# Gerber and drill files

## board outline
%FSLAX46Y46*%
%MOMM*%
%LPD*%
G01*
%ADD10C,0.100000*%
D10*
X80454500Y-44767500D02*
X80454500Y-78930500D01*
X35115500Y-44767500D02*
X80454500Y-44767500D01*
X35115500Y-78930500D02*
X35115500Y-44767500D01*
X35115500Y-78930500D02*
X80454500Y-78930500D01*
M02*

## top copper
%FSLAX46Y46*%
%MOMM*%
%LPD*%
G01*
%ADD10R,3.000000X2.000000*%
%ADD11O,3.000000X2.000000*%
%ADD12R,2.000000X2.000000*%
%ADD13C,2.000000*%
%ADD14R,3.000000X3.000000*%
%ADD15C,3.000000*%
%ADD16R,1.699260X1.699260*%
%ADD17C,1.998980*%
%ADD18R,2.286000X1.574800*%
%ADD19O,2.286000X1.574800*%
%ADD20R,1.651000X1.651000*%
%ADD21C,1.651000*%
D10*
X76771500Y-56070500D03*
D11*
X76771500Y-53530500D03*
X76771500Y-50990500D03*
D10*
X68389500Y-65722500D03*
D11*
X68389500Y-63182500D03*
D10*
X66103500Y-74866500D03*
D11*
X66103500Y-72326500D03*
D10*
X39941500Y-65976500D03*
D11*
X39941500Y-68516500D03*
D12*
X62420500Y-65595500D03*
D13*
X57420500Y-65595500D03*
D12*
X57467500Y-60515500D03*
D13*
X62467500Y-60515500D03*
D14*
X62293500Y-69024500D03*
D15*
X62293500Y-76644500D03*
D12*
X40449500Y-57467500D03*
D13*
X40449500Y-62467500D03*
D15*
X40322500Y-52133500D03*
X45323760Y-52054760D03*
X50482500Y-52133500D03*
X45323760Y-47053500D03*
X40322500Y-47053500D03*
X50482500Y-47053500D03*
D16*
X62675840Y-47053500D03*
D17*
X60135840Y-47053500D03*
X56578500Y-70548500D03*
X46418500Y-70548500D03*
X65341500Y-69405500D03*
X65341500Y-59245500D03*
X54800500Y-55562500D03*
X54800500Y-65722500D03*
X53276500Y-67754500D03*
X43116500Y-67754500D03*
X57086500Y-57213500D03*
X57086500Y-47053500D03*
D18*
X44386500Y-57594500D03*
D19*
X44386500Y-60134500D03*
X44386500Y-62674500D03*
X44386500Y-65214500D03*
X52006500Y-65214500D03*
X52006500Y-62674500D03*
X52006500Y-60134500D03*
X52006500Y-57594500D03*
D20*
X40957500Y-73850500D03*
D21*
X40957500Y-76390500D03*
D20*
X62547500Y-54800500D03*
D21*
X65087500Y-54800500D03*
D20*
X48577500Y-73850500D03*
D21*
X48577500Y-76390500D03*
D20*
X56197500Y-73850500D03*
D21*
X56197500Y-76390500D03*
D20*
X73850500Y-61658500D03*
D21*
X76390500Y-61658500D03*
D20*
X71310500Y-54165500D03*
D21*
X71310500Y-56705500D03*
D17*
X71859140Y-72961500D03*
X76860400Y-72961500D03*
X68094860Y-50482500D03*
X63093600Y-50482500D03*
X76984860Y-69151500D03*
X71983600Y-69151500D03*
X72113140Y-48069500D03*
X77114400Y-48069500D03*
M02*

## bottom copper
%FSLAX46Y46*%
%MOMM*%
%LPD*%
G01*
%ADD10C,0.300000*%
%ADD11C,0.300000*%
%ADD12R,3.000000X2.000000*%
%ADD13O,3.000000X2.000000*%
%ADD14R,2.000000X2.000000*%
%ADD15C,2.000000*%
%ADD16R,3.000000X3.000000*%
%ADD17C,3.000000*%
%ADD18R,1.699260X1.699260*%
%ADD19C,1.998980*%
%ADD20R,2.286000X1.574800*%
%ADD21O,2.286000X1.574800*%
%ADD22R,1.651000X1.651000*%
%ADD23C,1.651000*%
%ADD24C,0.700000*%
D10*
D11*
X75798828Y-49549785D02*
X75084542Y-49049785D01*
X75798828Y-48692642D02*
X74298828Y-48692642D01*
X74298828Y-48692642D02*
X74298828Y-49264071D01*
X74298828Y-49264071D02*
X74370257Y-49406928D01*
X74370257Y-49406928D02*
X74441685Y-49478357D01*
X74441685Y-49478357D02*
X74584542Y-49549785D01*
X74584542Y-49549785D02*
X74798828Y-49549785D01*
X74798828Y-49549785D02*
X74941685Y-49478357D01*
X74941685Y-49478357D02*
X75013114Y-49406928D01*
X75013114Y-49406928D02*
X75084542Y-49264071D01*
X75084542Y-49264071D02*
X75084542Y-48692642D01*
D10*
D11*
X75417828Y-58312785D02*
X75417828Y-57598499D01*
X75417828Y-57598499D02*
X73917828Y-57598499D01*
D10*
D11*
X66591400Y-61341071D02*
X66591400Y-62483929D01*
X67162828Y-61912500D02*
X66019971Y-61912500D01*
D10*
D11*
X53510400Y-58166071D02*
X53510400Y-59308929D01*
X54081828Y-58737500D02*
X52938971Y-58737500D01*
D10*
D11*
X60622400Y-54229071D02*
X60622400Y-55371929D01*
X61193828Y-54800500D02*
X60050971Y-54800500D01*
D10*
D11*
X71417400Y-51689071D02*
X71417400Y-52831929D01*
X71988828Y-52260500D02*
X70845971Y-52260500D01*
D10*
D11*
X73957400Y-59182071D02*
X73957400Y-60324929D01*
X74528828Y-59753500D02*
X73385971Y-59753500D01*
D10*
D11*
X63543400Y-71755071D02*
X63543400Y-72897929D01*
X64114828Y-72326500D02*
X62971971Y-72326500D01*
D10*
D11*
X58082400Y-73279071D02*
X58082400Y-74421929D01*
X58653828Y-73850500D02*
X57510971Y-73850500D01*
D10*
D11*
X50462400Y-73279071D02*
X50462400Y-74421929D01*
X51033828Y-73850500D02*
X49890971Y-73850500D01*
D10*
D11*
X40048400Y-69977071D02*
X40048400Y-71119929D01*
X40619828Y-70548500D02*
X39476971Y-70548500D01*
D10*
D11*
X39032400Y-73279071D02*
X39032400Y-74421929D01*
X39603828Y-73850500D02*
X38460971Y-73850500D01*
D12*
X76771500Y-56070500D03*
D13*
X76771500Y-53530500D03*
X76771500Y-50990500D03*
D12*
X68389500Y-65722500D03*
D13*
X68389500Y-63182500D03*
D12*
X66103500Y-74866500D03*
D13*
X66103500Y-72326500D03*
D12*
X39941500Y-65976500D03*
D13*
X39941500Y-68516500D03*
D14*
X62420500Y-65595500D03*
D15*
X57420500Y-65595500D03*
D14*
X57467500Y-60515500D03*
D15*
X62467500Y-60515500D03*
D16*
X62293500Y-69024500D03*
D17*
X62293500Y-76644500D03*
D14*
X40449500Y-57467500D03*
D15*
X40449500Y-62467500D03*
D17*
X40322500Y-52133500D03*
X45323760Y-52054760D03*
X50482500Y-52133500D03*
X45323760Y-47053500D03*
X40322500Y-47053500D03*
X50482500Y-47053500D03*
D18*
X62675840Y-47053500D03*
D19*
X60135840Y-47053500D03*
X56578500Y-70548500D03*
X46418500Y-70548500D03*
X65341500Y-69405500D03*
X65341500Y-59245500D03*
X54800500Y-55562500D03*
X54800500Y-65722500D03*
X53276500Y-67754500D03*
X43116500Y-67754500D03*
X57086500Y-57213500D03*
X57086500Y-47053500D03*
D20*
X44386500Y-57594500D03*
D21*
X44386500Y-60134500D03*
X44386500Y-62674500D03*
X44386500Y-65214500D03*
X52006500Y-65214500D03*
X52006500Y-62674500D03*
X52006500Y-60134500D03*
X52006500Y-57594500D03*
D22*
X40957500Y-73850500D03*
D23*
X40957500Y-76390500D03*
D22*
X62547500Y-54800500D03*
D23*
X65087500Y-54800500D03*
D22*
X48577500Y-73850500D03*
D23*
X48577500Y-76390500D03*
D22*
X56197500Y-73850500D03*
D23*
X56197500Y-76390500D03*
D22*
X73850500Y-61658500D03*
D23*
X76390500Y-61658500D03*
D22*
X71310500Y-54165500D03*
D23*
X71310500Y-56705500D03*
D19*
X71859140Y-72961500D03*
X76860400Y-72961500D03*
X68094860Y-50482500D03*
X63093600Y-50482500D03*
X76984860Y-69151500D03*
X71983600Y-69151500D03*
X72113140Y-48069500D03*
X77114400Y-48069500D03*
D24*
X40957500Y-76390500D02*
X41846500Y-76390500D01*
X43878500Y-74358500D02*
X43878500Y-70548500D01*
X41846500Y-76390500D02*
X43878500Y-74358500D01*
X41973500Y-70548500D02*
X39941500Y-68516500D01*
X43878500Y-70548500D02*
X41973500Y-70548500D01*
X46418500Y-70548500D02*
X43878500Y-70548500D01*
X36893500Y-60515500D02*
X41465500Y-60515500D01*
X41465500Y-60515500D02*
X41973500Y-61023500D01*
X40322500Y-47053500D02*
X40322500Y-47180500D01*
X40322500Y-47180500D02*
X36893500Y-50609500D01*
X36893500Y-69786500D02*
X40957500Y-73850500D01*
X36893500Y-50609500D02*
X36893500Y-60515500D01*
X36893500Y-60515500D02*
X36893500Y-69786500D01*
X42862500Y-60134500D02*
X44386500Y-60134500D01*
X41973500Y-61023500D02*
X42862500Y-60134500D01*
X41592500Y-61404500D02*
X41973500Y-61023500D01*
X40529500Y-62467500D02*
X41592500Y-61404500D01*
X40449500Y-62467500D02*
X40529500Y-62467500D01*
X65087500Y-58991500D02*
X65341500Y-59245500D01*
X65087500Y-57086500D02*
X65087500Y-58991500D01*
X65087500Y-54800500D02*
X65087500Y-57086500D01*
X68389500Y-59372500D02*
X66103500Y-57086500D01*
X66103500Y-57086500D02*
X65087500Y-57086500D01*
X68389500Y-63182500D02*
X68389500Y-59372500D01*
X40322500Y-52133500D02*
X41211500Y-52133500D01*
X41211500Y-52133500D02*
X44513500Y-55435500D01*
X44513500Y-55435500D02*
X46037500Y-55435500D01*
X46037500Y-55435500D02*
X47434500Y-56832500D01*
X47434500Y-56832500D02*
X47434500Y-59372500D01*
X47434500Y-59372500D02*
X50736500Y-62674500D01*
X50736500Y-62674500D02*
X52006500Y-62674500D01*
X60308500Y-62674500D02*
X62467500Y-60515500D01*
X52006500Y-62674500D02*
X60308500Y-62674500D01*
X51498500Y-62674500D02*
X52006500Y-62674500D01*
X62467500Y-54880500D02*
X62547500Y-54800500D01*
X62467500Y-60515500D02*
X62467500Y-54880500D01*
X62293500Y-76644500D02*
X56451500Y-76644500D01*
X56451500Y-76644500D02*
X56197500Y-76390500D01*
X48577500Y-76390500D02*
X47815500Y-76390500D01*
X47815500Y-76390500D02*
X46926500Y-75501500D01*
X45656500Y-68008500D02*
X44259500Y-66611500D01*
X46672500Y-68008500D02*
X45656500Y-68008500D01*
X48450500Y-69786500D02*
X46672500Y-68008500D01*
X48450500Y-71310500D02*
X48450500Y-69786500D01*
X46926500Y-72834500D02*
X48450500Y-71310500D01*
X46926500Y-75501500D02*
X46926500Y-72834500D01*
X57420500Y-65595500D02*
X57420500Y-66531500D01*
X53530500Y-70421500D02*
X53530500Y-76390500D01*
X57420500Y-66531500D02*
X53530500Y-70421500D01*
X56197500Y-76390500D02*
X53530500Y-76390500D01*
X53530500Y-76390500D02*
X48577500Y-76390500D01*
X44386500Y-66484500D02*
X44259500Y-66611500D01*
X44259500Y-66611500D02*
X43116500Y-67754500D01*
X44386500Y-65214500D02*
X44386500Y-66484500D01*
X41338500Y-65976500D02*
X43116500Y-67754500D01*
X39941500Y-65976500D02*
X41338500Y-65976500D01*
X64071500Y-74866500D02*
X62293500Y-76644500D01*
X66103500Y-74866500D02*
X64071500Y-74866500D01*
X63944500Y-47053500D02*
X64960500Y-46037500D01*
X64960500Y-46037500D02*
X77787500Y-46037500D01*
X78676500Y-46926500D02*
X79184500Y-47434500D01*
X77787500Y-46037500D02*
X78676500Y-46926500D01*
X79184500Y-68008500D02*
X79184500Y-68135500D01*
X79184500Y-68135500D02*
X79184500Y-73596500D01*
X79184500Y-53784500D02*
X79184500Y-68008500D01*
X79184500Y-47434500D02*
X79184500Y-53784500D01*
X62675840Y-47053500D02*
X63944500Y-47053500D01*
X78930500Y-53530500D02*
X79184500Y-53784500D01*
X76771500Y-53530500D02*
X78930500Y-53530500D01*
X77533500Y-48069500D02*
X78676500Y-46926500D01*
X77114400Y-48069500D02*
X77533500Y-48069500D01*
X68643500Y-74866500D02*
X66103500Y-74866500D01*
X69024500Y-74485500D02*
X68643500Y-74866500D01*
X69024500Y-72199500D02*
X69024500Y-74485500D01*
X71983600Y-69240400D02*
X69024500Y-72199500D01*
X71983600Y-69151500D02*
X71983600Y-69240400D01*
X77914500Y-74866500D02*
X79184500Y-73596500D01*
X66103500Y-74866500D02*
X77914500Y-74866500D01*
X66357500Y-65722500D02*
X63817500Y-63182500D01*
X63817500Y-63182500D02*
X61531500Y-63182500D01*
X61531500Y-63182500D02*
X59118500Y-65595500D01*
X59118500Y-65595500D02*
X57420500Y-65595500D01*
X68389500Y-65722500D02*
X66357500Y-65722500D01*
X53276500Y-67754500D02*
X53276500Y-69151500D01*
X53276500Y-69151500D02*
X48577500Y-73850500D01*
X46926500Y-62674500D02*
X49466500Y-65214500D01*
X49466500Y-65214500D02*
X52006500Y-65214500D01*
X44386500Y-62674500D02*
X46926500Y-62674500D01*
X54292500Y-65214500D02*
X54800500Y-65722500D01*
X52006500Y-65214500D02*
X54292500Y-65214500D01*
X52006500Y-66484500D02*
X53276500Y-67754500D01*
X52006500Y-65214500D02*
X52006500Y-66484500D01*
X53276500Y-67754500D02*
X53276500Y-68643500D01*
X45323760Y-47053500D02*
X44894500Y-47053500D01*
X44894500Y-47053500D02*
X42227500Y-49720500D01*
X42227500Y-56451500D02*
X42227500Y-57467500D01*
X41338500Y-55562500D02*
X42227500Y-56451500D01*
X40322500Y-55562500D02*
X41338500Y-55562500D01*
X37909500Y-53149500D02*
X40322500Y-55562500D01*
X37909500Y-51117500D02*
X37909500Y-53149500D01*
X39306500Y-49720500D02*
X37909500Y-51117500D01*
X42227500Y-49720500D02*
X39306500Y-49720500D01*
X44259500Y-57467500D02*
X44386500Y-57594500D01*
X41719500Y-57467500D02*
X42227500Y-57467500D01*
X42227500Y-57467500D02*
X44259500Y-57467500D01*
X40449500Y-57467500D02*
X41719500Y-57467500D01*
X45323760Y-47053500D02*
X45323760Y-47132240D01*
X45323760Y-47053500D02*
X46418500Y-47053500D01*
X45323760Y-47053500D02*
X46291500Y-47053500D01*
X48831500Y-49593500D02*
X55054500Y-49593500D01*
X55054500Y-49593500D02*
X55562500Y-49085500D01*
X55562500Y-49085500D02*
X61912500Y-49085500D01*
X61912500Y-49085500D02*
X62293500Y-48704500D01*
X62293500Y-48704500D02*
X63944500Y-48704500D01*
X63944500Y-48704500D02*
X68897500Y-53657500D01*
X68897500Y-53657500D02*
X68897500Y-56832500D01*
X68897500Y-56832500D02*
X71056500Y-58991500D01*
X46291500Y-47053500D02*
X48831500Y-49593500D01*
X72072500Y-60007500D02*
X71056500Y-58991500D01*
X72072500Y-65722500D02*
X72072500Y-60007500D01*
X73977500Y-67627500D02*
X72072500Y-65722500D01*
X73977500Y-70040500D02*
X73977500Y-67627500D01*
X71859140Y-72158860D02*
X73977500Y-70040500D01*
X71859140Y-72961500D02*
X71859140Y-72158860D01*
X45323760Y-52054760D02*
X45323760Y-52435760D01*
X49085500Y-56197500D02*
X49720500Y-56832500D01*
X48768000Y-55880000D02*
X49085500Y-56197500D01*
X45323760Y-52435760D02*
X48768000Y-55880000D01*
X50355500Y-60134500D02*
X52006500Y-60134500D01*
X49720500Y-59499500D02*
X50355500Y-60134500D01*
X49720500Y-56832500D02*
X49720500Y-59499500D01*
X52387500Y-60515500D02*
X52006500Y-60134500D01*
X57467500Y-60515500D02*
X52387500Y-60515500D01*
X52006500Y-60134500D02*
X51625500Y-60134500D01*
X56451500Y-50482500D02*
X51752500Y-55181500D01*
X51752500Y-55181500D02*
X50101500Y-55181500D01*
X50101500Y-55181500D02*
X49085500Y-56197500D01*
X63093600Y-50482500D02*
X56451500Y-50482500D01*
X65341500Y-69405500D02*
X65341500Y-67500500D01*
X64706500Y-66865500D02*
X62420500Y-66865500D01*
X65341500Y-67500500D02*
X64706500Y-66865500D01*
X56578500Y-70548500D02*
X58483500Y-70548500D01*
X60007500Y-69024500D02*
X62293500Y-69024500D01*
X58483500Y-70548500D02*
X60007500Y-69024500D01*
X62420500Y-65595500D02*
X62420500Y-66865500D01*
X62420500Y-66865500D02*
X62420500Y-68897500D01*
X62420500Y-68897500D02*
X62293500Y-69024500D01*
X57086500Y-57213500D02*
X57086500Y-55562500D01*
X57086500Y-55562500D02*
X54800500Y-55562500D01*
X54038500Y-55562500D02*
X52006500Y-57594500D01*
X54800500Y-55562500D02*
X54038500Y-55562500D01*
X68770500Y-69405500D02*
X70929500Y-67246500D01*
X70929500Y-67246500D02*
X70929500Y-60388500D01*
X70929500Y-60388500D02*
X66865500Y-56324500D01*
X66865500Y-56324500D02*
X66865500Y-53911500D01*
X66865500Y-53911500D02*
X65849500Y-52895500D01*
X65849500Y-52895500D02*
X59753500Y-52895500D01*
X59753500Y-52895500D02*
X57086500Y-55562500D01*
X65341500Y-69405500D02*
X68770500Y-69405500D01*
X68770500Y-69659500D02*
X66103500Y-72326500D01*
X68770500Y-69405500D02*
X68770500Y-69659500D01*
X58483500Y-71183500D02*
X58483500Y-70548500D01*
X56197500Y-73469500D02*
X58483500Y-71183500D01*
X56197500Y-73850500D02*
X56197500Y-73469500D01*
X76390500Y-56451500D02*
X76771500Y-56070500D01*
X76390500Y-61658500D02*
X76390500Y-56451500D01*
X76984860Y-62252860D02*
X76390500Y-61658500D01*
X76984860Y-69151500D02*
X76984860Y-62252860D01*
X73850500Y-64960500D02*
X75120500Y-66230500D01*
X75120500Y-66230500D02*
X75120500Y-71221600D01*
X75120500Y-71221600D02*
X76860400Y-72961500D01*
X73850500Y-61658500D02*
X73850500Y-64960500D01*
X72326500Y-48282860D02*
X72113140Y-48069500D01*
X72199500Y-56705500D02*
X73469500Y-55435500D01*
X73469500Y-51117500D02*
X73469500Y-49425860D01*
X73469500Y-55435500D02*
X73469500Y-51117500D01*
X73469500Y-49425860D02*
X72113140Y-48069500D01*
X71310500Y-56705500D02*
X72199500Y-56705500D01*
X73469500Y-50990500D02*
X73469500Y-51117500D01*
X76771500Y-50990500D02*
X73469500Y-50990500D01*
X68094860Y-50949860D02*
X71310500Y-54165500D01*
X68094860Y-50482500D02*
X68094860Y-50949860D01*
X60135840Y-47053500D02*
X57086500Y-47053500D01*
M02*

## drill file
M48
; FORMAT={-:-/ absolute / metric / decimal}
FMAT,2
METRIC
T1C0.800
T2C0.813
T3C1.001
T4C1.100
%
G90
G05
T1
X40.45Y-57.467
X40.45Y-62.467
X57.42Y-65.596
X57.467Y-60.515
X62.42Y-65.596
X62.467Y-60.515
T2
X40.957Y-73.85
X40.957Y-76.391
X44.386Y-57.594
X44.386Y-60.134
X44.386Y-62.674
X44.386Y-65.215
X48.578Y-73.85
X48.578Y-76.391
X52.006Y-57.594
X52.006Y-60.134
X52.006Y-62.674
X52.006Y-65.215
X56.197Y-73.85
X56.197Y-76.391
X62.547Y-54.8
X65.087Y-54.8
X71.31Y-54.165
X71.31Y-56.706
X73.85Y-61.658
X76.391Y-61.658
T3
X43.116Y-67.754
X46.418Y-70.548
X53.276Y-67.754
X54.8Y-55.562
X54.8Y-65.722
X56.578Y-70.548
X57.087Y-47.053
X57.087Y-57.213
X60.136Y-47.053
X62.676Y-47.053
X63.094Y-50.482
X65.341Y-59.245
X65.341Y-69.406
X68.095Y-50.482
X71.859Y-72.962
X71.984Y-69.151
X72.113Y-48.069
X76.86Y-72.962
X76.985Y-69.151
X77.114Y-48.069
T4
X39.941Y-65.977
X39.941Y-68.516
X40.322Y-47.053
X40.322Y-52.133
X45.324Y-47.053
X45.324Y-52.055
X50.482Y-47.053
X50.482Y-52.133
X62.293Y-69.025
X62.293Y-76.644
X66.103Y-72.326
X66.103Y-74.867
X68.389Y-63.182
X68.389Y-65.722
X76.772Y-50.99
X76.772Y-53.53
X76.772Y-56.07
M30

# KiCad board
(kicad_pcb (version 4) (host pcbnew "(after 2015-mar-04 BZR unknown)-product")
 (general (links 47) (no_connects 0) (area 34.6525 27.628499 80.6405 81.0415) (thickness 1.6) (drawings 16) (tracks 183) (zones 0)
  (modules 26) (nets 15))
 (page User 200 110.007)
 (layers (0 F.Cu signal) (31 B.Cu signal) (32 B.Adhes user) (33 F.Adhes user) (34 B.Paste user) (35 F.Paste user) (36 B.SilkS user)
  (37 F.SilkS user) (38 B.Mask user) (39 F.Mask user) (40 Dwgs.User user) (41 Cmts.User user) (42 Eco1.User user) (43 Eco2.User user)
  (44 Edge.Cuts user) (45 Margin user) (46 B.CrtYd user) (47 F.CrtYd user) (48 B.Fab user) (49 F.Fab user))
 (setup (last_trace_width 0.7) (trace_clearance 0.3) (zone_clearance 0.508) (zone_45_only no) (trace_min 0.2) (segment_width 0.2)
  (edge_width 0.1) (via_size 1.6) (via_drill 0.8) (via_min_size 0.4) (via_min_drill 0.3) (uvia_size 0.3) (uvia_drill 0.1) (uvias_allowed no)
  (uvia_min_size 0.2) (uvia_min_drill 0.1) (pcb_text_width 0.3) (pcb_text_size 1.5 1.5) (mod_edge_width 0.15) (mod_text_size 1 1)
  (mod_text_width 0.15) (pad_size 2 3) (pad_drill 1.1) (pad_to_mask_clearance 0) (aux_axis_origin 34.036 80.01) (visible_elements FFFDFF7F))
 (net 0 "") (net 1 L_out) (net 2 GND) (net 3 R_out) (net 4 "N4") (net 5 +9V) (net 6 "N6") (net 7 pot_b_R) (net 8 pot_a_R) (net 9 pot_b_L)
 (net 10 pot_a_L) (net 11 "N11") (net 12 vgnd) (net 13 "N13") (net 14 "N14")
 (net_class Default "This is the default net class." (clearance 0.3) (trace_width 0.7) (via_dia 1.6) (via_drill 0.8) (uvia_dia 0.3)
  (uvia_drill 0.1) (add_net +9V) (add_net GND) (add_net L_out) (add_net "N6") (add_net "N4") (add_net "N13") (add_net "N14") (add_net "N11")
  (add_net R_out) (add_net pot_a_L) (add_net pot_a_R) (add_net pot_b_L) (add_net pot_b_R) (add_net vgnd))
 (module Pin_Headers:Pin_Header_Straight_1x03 (layer F.Cu) (at 76.7715 56.0705 180)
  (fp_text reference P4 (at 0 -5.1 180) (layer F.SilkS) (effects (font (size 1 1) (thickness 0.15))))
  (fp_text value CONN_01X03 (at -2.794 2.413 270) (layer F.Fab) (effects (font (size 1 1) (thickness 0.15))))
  (pad 1 thru_hole rect (at 0 0 180) (size 3 2) (drill 1.1) (layers *.Cu *.Mask F.SilkS) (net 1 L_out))
  (pad 2 thru_hole oval (at 0 2.54 180) (size 3 2) (drill 1.1) (layers *.Cu *.Mask F.SilkS) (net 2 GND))
  (pad 3 thru_hole oval (at 0 5.08 180) (size 3 2) (drill 1.1) (layers *.Cu *.Mask F.SilkS) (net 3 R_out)))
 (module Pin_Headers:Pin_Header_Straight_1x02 (layer F.Cu) (at 68.3895 65.7225 180)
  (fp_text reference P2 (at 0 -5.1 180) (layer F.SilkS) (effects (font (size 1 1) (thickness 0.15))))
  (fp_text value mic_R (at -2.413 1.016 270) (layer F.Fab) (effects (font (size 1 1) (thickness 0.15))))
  (pad 1 thru_hole rect (at 0 0 180) (size 3 2) (drill 1.1) (layers *.Cu *.Mask F.SilkS) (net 2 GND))
  (pad 2 thru_hole oval (at 0 2.54 180) (size 3 2) (drill 1.1) (layers *.Cu *.Mask F.SilkS) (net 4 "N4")))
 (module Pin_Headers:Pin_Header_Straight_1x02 (layer F.Cu) (at 66.1035 74.8665 180)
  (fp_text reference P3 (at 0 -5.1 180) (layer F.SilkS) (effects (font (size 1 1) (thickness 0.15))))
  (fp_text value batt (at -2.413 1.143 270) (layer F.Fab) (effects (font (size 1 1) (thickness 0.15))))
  (pad 1 thru_hole rect (at 0 0 180) (size 3 2) (drill 1.1) (layers *.Cu *.Mask F.SilkS) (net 2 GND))
  (pad 2 thru_hole oval (at 0 2.54 180) (size 3 2) (drill 1.1) (layers *.Cu *.Mask F.SilkS) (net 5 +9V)))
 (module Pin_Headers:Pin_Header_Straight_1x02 (layer F.Cu) (at 39.9415 65.9765)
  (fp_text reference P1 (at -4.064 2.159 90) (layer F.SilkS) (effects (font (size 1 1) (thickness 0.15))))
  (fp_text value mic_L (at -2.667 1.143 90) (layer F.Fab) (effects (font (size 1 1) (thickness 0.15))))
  (pad 1 thru_hole rect (at 0 0) (size 3 2) (drill 1.1) (layers *.Cu *.Mask F.SilkS) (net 2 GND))
  (pad 2 thru_hole oval (at 0 2.54) (size 3 2) (drill 1.1) (layers *.Cu *.Mask F.SilkS) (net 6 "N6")))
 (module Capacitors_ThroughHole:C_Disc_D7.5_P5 (layer F.Cu) (at 62.4205 65.5955 180)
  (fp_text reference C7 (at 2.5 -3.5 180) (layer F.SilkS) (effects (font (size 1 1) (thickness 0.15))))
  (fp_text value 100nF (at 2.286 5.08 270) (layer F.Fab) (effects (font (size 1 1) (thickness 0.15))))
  (pad 1 thru_hole rect (at 0 0 180) (size 2 2) (drill 0.8) (layers *.Cu *.Mask F.SilkS) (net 5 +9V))
  (pad 2 thru_hole circle (at 5 0 180) (size 2 2) (drill 0.8) (layers *.Cu *.Mask F.SilkS) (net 2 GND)))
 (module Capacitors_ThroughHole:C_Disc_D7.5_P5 (layer F.Cu) (at 57.4675 60.5155)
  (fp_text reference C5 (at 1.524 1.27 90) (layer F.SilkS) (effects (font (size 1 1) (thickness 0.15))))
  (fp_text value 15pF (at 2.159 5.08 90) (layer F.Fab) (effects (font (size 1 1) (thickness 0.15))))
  (pad 1 thru_hole rect (at 0 0) (size 2 2) (drill 0.8) (layers *.Cu *.Mask F.SilkS) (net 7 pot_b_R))
  (pad 2 thru_hole circle (at 5 0) (size 2 2) (drill 0.8) (layers *.Cu *.Mask F.SilkS) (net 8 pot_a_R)))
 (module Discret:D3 (layer F.Cu) (at 62.2935 72.8345 90)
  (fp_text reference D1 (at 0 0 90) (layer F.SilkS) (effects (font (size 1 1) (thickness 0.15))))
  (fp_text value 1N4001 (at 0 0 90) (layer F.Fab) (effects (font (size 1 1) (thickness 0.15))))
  (pad 1 thru_hole rect (at 3.81 0 90) (size 3 3) (drill 1.1) (layers *.Cu *.Mask F.SilkS) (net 5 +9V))
  (pad 2 thru_hole circle (at -3.81 0 90) (size 3 3) (drill 1.1) (layers *.Cu *.Mask F.SilkS) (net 2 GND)))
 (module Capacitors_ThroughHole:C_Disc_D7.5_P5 (layer F.Cu) (at 40.4495 57.4675 270)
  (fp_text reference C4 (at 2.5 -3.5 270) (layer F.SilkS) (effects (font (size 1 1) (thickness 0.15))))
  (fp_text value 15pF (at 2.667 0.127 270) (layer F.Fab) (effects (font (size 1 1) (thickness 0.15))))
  (pad 1 thru_hole rect (at 0 0 270) (size 2 2) (drill 0.8) (layers *.Cu *.Mask F.SilkS) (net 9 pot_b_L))
  (pad 2 thru_hole circle (at 5 0 270) (size 2 2) (drill 0.8) (layers *.Cu *.Mask F.SilkS) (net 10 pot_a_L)))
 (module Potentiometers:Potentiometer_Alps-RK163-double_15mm (layer F.Cu) (at 50.4825 47.0535 90)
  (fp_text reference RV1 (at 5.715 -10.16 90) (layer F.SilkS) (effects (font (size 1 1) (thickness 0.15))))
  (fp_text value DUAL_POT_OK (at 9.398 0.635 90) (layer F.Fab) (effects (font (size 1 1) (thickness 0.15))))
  (pad 23 thru_hole circle (at -5.08 -10.16 90) (size 3 3) (drill 1.1) (layers *.Cu *.Mask F.SilkS) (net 8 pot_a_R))
  (pad 22 thru_hole circle (at -5.00126 -5.15874 90) (size 3 3) (drill 1.1) (layers *.Cu *.Mask F.SilkS) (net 7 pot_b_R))
  (pad 21 thru_hole circle (at -5.08 0 90) (size 3 3) (drill 1.1) (layers *.Cu *.Mask F.SilkS))
  (pad 12 thru_hole circle (at 0 -5.15874 90) (size 3 3) (drill 1.1) (layers *.Cu *.Mask F.SilkS) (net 9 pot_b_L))
  (pad 13 thru_hole circle (at 0 -10.16 90) (size 3 3) (drill 1.1) (layers *.Cu *.Mask F.SilkS) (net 10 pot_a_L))
  (pad 11 thru_hole circle (at 0 0 90) (size 3 3) (drill 1.1) (layers *.Cu *.Mask F.SilkS)))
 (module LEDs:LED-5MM (layer F.Cu) (at 62.6745 47.0535 180)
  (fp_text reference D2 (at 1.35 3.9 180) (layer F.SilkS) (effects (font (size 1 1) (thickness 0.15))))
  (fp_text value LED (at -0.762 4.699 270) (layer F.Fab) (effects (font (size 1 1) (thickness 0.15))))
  (pad 1 thru_hole rect (at -0.00134 0 270) (size 1.69926 1.69926) (drill 1.00076) (layers *.Cu *.Mask F.SilkS) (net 2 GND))
  (pad 2 thru_hole circle (at 2.53866 0 180) (size 1.99898 1.99898) (drill 1.00076) (layers *.Cu *.Mask F.SilkS) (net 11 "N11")))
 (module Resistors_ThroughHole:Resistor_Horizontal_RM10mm (layer F.Cu) (at 51.4985 70.5485 180)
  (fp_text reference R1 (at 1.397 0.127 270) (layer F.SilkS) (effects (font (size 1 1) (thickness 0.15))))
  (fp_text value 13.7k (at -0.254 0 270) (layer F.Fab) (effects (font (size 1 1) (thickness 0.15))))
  (pad 1 thru_hole circle (at -5.08 0 180) (size 1.99898 1.99898) (drill 1.00076) (layers *.Cu *.SilkS *.Mask) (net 5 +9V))
  (pad 2 thru_hole circle (at 5.08 0 180) (size 1.99898 1.99898) (drill 1.00076) (layers *.Cu *.SilkS *.Mask) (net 6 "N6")))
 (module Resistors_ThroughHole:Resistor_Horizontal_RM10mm (layer F.Cu) (at 65.3415 64.3255 90)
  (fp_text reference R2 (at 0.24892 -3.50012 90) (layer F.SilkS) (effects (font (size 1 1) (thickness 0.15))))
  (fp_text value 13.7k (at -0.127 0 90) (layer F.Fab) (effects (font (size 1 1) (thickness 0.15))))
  (pad 1 thru_hole circle (at -5.08 0 90) (size 1.99898 1.99898) (drill 1.00076) (layers *.Cu *.SilkS *.Mask) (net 5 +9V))
  (pad 2 thru_hole circle (at 5.08 0 90) (size 1.99898 1.99898) (drill 1.00076) (layers *.Cu *.SilkS *.Mask) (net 4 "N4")))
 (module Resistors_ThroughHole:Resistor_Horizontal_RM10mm (layer F.Cu) (at 54.8005 60.6425 270)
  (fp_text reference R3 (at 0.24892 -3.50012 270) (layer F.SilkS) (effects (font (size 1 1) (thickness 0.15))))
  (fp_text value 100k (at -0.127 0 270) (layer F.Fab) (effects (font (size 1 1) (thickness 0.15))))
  (pad 1 thru_hole circle (at -5.08 0 270) (size 1.99898 1.99898) (drill 1.00076) (layers *.Cu *.SilkS *.Mask) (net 5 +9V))
  (pad 2 thru_hole circle (at 5.08 0 270) (size 1.99898 1.99898) (drill 1.00076) (layers *.Cu *.SilkS *.Mask) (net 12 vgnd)))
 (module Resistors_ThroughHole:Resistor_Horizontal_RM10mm (layer F.Cu) (at 48.1965 67.7545 180)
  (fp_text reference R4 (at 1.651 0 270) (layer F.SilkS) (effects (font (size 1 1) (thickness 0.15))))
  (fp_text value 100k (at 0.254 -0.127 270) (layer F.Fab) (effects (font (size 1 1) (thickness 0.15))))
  (pad 1 thru_hole circle (at -5.08 0 180) (size 1.99898 1.99898) (drill 1.00076) (layers *.Cu *.SilkS *.Mask) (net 12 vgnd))
  (pad 2 thru_hole circle (at 5.08 0 180) (size 1.99898 1.99898) (drill 1.00076) (layers *.Cu *.SilkS *.Mask) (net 2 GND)))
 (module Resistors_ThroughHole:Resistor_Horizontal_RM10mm (layer F.Cu) (at 57.0865 52.1335 90)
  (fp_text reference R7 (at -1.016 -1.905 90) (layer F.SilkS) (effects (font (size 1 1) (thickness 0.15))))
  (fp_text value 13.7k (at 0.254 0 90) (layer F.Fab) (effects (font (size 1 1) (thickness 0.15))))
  (pad 1 thru_hole circle (at -5.08 0 90) (size 1.99898 1.99898) (drill 1.00076) (layers *.Cu *.SilkS *.Mask) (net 5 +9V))
  (pad 2 thru_hole circle (at 5.08 0 90) (size 1.99898 1.99898) (drill 1.00076) (layers *.Cu *.SilkS *.Mask) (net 11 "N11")))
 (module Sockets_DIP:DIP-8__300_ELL (layer F.Cu) (at 48.1965 61.4045 270)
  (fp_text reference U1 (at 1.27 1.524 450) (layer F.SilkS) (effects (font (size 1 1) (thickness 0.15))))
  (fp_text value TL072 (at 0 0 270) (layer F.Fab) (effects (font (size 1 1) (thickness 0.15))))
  (pad 1 thru_hole rect (at -3.81 3.81 270) (size 1.5748 2.286) (drill 0.8128) (layers *.Cu *.Mask F.SilkS) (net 9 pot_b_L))
  (pad 2 thru_hole oval (at -1.27 3.81 270) (size 1.5748 2.286) (drill 0.8128) (layers *.Cu *.Mask F.SilkS) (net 10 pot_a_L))
  (pad 3 thru_hole oval (at 1.27 3.81 270) (size 1.5748 2.286) (drill 0.8128) (layers *.Cu *.Mask F.SilkS) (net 12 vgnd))
  (pad 4 thru_hole oval (at 3.81 3.81 270) (size 1.5748 2.286) (drill 0.8128) (layers *.Cu *.Mask F.SilkS) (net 2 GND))
  (pad 5 thru_hole oval (at 3.81 -3.81 270) (size 1.5748 2.286) (drill 0.8128) (layers *.Cu *.Mask F.SilkS) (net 12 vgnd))
  (pad 6 thru_hole oval (at 1.27 -3.81 270) (size 1.5748 2.286) (drill 0.8128) (layers *.Cu *.Mask F.SilkS) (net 8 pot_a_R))
  (pad 7 thru_hole oval (at -1.27 -3.81 270) (size 1.5748 2.286) (drill 0.8128) (layers *.Cu *.Mask F.SilkS) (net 7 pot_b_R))
  (pad 8 thru_hole oval (at -3.81 -3.81 270) (size 1.5748 2.286) (drill 0.8128) (layers *.Cu *.Mask F.SilkS) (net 5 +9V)))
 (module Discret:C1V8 (layer F.Cu) (at 40.9575 75.1205 270)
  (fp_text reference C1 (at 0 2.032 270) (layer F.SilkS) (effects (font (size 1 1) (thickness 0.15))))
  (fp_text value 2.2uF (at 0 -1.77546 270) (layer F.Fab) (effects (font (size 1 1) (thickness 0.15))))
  (pad 1 thru_hole rect (at -1.27 0 270) (size 1.651 1.651) (drill 0.8128) (layers *.Cu *.Mask F.SilkS) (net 10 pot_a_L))
  (pad 2 thru_hole circle (at 1.27 0 270) (size 1.651 1.651) (drill 0.8128) (layers *.Cu *.Mask F.SilkS) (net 6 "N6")))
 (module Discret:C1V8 (layer F.Cu) (at 63.8175 54.8005)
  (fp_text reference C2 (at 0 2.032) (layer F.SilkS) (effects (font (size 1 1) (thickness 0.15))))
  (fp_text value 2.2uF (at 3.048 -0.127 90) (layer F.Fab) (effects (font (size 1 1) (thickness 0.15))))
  (pad 1 thru_hole rect (at -1.27 0) (size 1.651 1.651) (drill 0.8128) (layers *.Cu *.Mask F.SilkS) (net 8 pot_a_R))
  (pad 2 thru_hole circle (at 1.27 0) (size 1.651 1.651) (drill 0.8128) (layers *.Cu *.Mask F.SilkS) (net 4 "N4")))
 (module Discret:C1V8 (layer F.Cu) (at 48.5775 75.1205 270)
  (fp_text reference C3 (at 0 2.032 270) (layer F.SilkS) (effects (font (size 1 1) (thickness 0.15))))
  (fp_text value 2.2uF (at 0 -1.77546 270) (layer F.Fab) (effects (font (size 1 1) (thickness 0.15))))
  (pad 1 thru_hole rect (at -1.27 0 270) (size 1.651 1.651) (drill 0.8128) (layers *.Cu *.Mask F.SilkS) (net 12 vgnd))
  (pad 2 thru_hole circle (at 1.27 0 270) (size 1.651 1.651) (drill 0.8128) (layers *.Cu *.Mask F.SilkS) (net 2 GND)))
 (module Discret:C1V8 (layer F.Cu) (at 56.1975 75.1205 270)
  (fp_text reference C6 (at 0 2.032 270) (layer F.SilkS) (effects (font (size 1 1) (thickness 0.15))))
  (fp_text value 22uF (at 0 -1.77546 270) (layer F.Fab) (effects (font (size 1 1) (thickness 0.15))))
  (pad 1 thru_hole rect (at -1.27 0 270) (size 1.651 1.651) (drill 0.8128) (layers *.Cu *.Mask F.SilkS) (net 5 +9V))
  (pad 2 thru_hole circle (at 1.27 0 270) (size 1.651 1.651) (drill 0.8128) (layers *.Cu *.Mask F.SilkS) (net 2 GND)))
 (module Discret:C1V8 (layer F.Cu) (at 75.1205 61.6585)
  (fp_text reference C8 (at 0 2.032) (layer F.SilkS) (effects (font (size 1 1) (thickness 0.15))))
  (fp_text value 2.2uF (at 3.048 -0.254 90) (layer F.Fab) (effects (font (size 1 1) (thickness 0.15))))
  (pad 1 thru_hole rect (at -1.27 0) (size 1.651 1.651) (drill 0.8128) (layers *.Cu *.Mask F.SilkS) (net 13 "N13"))
  (pad 2 thru_hole circle (at 1.27 0) (size 1.651 1.651) (drill 0.8128) (layers *.Cu *.Mask F.SilkS) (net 1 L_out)))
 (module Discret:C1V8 (layer F.Cu) (at 71.3105 55.4355 270)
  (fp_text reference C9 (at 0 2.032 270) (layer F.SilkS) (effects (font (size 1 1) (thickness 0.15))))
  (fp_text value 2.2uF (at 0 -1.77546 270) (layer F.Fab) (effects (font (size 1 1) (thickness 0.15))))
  (pad 1 thru_hole rect (at -1.27 0 270) (size 1.651 1.651) (drill 0.8128) (layers *.Cu *.Mask F.SilkS) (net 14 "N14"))
  (pad 2 thru_hole circle (at 1.27 0 270) (size 1.651 1.651) (drill 0.8128) (layers *.Cu *.Mask F.SilkS) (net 3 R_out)))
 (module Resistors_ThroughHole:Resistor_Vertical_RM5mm (layer F.Cu) (at 74.3585 72.9615)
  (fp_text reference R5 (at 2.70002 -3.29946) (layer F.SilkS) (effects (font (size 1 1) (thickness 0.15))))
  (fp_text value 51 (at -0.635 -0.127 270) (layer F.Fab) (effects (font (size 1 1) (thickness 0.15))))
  (pad 1 thru_hole circle (at -2.49936 0) (size 1.99898 1.99898) (drill 1.00076) (layers *.Cu *.SilkS *.Mask) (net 9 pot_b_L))
  (pad 2 thru_hole circle (at 2.5019 0) (size 1.99898 1.99898) (drill 1.00076) (layers *.Cu *.SilkS *.Mask) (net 13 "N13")))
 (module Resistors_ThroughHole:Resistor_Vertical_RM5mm (layer F.Cu) (at 65.5955 50.4825 180)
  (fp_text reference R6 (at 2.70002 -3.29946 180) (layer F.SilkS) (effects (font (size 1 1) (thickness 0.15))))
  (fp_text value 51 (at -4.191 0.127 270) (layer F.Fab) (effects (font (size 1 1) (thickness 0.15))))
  (pad 1 thru_hole circle (at -2.49936 0 180) (size 1.99898 1.99898) (drill 1.00076) (layers *.Cu *.SilkS *.Mask) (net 14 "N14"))
  (pad 2 thru_hole circle (at 2.5019 0 180) (size 1.99898 1.99898) (drill 1.00076) (layers *.Cu *.SilkS *.Mask) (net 7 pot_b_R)))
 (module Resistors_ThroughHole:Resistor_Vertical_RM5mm (layer F.Cu) (at 74.4855 69.1515 180)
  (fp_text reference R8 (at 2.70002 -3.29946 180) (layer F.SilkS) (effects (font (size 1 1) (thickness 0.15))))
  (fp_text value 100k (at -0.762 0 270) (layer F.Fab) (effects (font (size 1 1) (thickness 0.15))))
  (pad 1 thru_hole circle (at -2.49936 0 180) (size 1.99898 1.99898) (drill 1.00076) (layers *.Cu *.SilkS *.Mask) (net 1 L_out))
  (pad 2 thru_hole circle (at 2.5019 0 180) (size 1.99898 1.99898) (drill 1.00076) (layers *.Cu *.SilkS *.Mask) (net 2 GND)))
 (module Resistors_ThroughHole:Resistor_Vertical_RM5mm (layer F.Cu) (at 74.6125 48.0695)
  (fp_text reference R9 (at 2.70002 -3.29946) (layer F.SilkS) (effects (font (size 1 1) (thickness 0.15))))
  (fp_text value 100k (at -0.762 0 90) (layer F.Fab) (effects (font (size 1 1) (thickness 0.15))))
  (pad 1 thru_hole circle (at -2.49936 0) (size 1.99898 1.99898) (drill 1.00076) (layers *.Cu *.SilkS *.Mask) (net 3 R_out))
  (pad 2 thru_hole circle (at 2.5019 0) (size 1.99898 1.99898) (drill 1.00076) (layers *.Cu *.SilkS *.Mask) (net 2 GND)))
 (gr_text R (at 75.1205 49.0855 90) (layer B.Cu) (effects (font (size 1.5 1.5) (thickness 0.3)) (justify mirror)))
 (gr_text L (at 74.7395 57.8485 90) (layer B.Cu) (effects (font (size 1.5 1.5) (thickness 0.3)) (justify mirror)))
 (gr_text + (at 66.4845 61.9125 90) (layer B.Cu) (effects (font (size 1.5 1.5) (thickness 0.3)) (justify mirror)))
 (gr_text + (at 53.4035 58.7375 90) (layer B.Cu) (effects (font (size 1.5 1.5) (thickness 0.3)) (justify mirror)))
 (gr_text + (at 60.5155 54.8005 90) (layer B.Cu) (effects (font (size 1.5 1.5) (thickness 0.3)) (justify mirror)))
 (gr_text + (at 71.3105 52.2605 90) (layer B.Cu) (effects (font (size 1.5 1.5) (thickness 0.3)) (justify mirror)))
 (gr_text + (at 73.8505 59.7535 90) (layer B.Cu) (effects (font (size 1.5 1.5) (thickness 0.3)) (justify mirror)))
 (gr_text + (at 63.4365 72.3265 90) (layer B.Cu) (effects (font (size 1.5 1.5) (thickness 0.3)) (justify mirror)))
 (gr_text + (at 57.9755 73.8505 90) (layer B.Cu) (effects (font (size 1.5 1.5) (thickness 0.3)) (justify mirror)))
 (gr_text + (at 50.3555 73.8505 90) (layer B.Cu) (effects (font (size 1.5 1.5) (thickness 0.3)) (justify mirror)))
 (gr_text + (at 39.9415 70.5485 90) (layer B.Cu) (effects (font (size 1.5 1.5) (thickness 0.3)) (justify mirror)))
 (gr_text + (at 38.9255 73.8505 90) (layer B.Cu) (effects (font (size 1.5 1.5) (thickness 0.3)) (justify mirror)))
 (gr_line (start 80.4545 44.7675) (end 80.4545 78.9305) (angle 90) (layer Edge.Cuts) (width 0.1))
 (gr_line (start 35.1155 44.7675) (end 80.4545 44.7675) (angle 90) (layer Edge.Cuts) (width 0.1))
 (gr_line (start 35.1155 78.9305) (end 35.1155 44.7675) (angle 90) (layer Edge.Cuts) (width 0.1))
 (gr_line (start 35.1155 78.9305) (end 80.4545 78.9305) (angle 90) (layer Edge.Cuts) (width 0.1))
 (segment (start 40.9575 76.3905) (end 41.8465 76.3905) (width 0.7) (layer B.Cu) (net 6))
 (segment (start 43.8785 74.3585) (end 43.8785 70.5485) (width 0.7) (layer B.Cu) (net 6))
 (segment (start 41.8465 76.3905) (end 43.8785 74.3585) (width 0.7) (layer B.Cu) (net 6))
 (segment (start 41.9735 70.5485) (end 39.9415 68.5165) (width 0.7) (layer B.Cu) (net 6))
 (segment (start 43.8785 70.5485) (end 41.9735 70.5485) (width 0.7) (layer B.Cu) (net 6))
 (segment (start 46.4185 70.5485) (end 43.8785 70.5485) (width 0.7) (layer B.Cu) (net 6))
 (segment (start 36.8935 60.5155) (end 41.4655 60.5155) (width 0.7) (layer B.Cu) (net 10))
 (segment (start 41.4655 60.5155) (end 41.9735 61.0235) (width 0.7) (layer B.Cu) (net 10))
 (segment (start 40.3225 47.0535) (end 40.3225 47.1805) (width 0.7) (layer B.Cu) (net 10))
 (segment (start 40.3225 47.1805) (end 36.8935 50.6095) (width 0.7) (layer B.Cu) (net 10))
 (segment (start 36.8935 69.7865) (end 40.9575 73.8505) (width 0.7) (layer B.Cu) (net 10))
 (segment (start 36.8935 50.6095) (end 36.8935 60.5155) (width 0.7) (layer B.Cu) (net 10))
 (segment (start 36.8935 60.5155) (end 36.8935 69.7865) (width 0.7) (layer B.Cu) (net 10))
 (segment (start 42.8625 60.1345) (end 44.3865 60.1345) (width 0.7) (layer B.Cu) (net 10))
 (segment (start 41.9735 61.0235) (end 42.8625 60.1345) (width 0.7) (layer B.Cu) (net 10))
 (segment (start 41.5925 61.4045) (end 41.9735 61.0235) (width 0.7) (layer B.Cu) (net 10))
 (segment (start 40.5295 62.4675) (end 41.5925 61.4045) (width 0.7) (layer B.Cu) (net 10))
 (segment (start 40.4495 62.4675) (end 40.5295 62.4675) (width 0.7) (layer B.Cu) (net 10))
 (segment (start 65.0875 58.9915) (end 65.3415 59.2455) (width 0.7) (layer B.Cu) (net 4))
 (segment (start 65.0875 57.0865) (end 65.0875 58.9915) (width 0.7) (layer B.Cu) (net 4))
 (segment (start 65.0875 54.8005) (end 65.0875 57.0865) (width 0.7) (layer B.Cu) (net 4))
 (segment (start 68.3895 59.3725) (end 66.1035 57.0865) (width 0.7) (layer B.Cu) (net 4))
 (segment (start 66.1035 57.0865) (end 65.0875 57.0865) (width 0.7) (layer B.Cu) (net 4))
 (segment (start 68.3895 63.1825) (end 68.3895 59.3725) (width 0.7) (layer B.Cu) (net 4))
 (segment (start 40.3225 52.1335) (end 41.2115 52.1335) (width 0.7) (layer B.Cu) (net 8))
 (segment (start 41.2115 52.1335) (end 44.5135 55.4355) (width 0.7) (layer B.Cu) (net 8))
 (segment (start 44.5135 55.4355) (end 46.0375 55.4355) (width 0.7) (layer B.Cu) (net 8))
 (segment (start 46.0375 55.4355) (end 47.4345 56.8325) (width 0.7) (layer B.Cu) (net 8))
 (segment (start 47.4345 56.8325) (end 47.4345 59.3725) (width 0.7) (layer B.Cu) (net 8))
 (segment (start 47.4345 59.3725) (end 50.7365 62.6745) (width 0.7) (layer B.Cu) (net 8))
 (segment (start 50.7365 62.6745) (end 52.0065 62.6745) (width 0.7) (layer B.Cu) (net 8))
 (segment (start 60.3085 62.6745) (end 62.4675 60.5155) (width 0.7) (layer B.Cu) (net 8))
 (segment (start 52.0065 62.6745) (end 60.3085 62.6745) (width 0.7) (layer B.Cu) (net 8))
 (segment (start 51.4985 62.6745) (end 52.0065 62.6745) (width 0.7) (layer B.Cu) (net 8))
 (segment (start 62.4675 54.8805) (end 62.5475 54.8005) (width 0.7) (layer B.Cu) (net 8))
 (segment (start 62.4675 60.5155) (end 62.4675 54.8805) (width 0.7) (layer B.Cu) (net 8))
 (segment (start 62.2935 76.6445) (end 56.4515 76.6445) (width 0.7) (layer B.Cu) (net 2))
 (segment (start 56.4515 76.6445) (end 56.1975 76.3905) (width 0.7) (layer B.Cu) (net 2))
 (segment (start 48.5775 76.3905) (end 47.8155 76.3905) (width 0.7) (layer B.Cu) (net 2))
 (segment (start 47.8155 76.3905) (end 46.9265 75.5015) (width 0.7) (layer B.Cu) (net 2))
 (segment (start 45.6565 68.0085) (end 44.2595 66.6115) (width 0.7) (layer B.Cu) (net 2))
 (segment (start 46.6725 68.0085) (end 45.6565 68.0085) (width 0.7) (layer B.Cu) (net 2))
 (segment (start 48.4505 69.7865) (end 46.6725 68.0085) (width 0.7) (layer B.Cu) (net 2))
 (segment (start 48.4505 71.3105) (end 48.4505 69.7865) (width 0.7) (layer B.Cu) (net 2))
 (segment (start 46.9265 72.8345) (end 48.4505 71.3105) (width 0.7) (layer B.Cu) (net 2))
 (segment (start 46.9265 75.5015) (end 46.9265 72.8345) (width 0.7) (layer B.Cu) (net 2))
 (segment (start 57.4205 65.5955) (end 57.4205 66.5315) (width 0.7) (layer B.Cu) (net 2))
 (segment (start 53.5305 70.4215) (end 53.5305 76.3905) (width 0.7) (layer B.Cu) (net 2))
 (segment (start 57.4205 66.5315) (end 53.5305 70.4215) (width 0.7) (layer B.Cu) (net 2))
 (segment (start 56.1975 76.3905) (end 53.5305 76.3905) (width 0.7) (layer B.Cu) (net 2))
 (segment (start 53.5305 76.3905) (end 48.5775 76.3905) (width 0.7) (layer B.Cu) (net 2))
 (segment (start 44.3865 66.4845) (end 44.2595 66.6115) (width 0.7) (layer B.Cu) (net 2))
 (segment (start 44.2595 66.6115) (end 43.1165 67.7545) (width 0.7) (layer B.Cu) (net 2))
 (segment (start 44.3865 65.2145) (end 44.3865 66.4845) (width 0.7) (layer B.Cu) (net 2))
 (segment (start 41.3385 65.9765) (end 43.1165 67.7545) (width 0.7) (layer B.Cu) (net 2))
 (segment (start 39.9415 65.9765) (end 41.3385 65.9765) (width 0.7) (layer B.Cu) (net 2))
 (segment (start 64.0715 74.8665) (end 62.2935 76.6445) (width 0.7) (layer B.Cu) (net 2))
 (segment (start 66.1035 74.8665) (end 64.0715 74.8665) (width 0.7) (layer B.Cu) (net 2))
 (segment (start 63.9445 47.0535) (end 64.9605 46.0375) (width 0.7) (layer B.Cu) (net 2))
 (segment (start 64.9605 46.0375) (end 77.7875 46.0375) (width 0.7) (layer B.Cu) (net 2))
 (segment (start 78.6765 46.9265) (end 79.1845 47.4345) (width 0.7) (layer B.Cu) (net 2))
 (segment (start 77.7875 46.0375) (end 78.6765 46.9265) (width 0.7) (layer B.Cu) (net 2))
 (segment (start 79.1845 68.0085) (end 79.1845 68.1355) (width 0.7) (layer B.Cu) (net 2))
 (segment (start 79.1845 68.1355) (end 79.1845 73.5965) (width 0.7) (layer B.Cu) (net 2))
 (segment (start 79.1845 53.7845) (end 79.1845 68.0085) (width 0.7) (layer B.Cu) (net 2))
 (segment (start 79.1845 47.4345) (end 79.1845 53.7845) (width 0.7) (layer B.Cu) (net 2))
 (segment (start 62.67584 47.0535) (end 63.9445 47.0535) (width 0.7) (layer B.Cu) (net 2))
 (segment (start 78.9305 53.5305) (end 79.1845 53.7845) (width 0.7) (layer B.Cu) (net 2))
 (segment (start 76.7715 53.5305) (end 78.9305 53.5305) (width 0.7) (layer B.Cu) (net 2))
 (segment (start 77.5335 48.0695) (end 78.6765 46.9265) (width 0.7) (layer B.Cu) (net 2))
 (segment (start 77.1144 48.0695) (end 77.5335 48.0695) (width 0.7) (layer B.Cu) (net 2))
 (segment (start 68.6435 74.8665) (end 66.1035 74.8665) (width 0.7) (layer B.Cu) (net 2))
 (segment (start 69.0245 74.4855) (end 68.6435 74.8665) (width 0.7) (layer B.Cu) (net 2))
 (segment (start 69.0245 72.1995) (end 69.0245 74.4855) (width 0.7) (layer B.Cu) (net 2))
 (segment (start 71.9836 69.2404) (end 69.0245 72.1995) (width 0.7) (layer B.Cu) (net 2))
 (segment (start 71.9836 69.1515) (end 71.9836 69.2404) (width 0.7) (layer B.Cu) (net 2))
 (segment (start 77.9145 74.8665) (end 79.1845 73.5965) (width 0.7) (layer B.Cu) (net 2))
 (segment (start 66.1035 74.8665) (end 77.9145 74.8665) (width 0.7) (layer B.Cu) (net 2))
 (segment (start 66.3575 65.7225) (end 63.8175 63.1825) (width 0.7) (layer B.Cu) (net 2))
 (segment (start 63.8175 63.1825) (end 61.5315 63.1825) (width 0.7) (layer B.Cu) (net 2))
 (segment (start 61.5315 63.1825) (end 59.1185 65.5955) (width 0.7) (layer B.Cu) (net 2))
 (segment (start 59.1185 65.5955) (end 57.4205 65.5955) (width 0.7) (layer B.Cu) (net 2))
 (segment (start 68.3895 65.7225) (end 66.3575 65.7225) (width 0.7) (layer B.Cu) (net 2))
 (segment (start 53.2765 67.7545) (end 53.2765 69.1515) (width 0.7) (layer B.Cu) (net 12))
 (segment (start 53.2765 69.1515) (end 48.5775 73.8505) (width 0.7) (layer B.Cu) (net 12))
 (segment (start 46.9265 62.6745) (end 49.4665 65.2145) (width 0.7) (layer B.Cu) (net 12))
 (segment (start 49.4665 65.2145) (end 52.0065 65.2145) (width 0.7) (layer B.Cu) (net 12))
 (segment (start 44.3865 62.6745) (end 46.9265 62.6745) (width 0.7) (layer B.Cu) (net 12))
 (segment (start 54.2925 65.2145) (end 54.8005 65.7225) (width 0.7) (layer B.Cu) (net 12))
 (segment (start 52.0065 65.2145) (end 54.2925 65.2145) (width 0.7) (layer B.Cu) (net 12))
 (segment (start 52.0065 66.4845) (end 53.2765 67.7545) (width 0.7) (layer B.Cu) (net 12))
 (segment (start 52.0065 65.2145) (end 52.0065 66.4845) (width 0.7) (layer B.Cu) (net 12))
 (segment (start 53.2765 67.7545) (end 53.2765 68.6435) (width 0.7) (layer B.Cu) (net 12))
 (segment (start 45.32376 47.0535) (end 44.8945 47.0535) (width 0.7) (layer B.Cu) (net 9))
 (segment (start 44.8945 47.0535) (end 42.2275 49.7205) (width 0.7) (layer B.Cu) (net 9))
 (segment (start 42.2275 56.4515) (end 42.2275 57.4675) (width 0.7) (layer B.Cu) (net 9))
 (segment (start 41.3385 55.5625) (end 42.2275 56.4515) (width 0.7) (layer B.Cu) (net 9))
 (segment (start 40.3225 55.5625) (end 41.3385 55.5625) (width 0.7) (layer B.Cu) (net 9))
 (segment (start 37.9095 53.1495) (end 40.3225 55.5625) (width 0.7) (layer B.Cu) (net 9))
 (segment (start 37.9095 51.1175) (end 37.9095 53.1495) (width 0.7) (layer B.Cu) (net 9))
 (segment (start 39.3065 49.7205) (end 37.9095 51.1175) (width 0.7) (layer B.Cu) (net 9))
 (segment (start 42.2275 49.7205) (end 39.3065 49.7205) (width 0.7) (layer B.Cu) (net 9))
 (segment (start 44.2595 57.4675) (end 44.3865 57.5945) (width 0.7) (layer B.Cu) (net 9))
 (segment (start 41.7195 57.4675) (end 42.2275 57.4675) (width 0.7) (layer B.Cu) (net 9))
 (segment (start 42.2275 57.4675) (end 44.2595 57.4675) (width 0.7) (layer B.Cu) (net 9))
 (segment (start 40.4495 57.4675) (end 41.7195 57.4675) (width 0.7) (layer B.Cu) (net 9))
 (segment (start 45.32376 47.0535) (end 45.32376 47.13224) (width 0.7) (layer B.Cu) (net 9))
 (segment (start 45.32376 47.0535) (end 46.4185 47.0535) (width 0.7) (layer B.Cu) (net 9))
 (segment (start 45.32376 47.0535) (end 46.2915 47.0535) (width 0.7) (layer B.Cu) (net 9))
 (segment (start 48.8315 49.5935) (end 55.0545 49.5935) (width 0.7) (layer B.Cu) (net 9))
 (segment (start 55.0545 49.5935) (end 55.5625 49.0855) (width 0.7) (layer B.Cu) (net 9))
 (segment (start 55.5625 49.0855) (end 61.9125 49.0855) (width 0.7) (layer B.Cu) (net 9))
 (segment (start 61.9125 49.0855) (end 62.2935 48.7045) (width 0.7) (layer B.Cu) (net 9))
 (segment (start 62.2935 48.7045) (end 63.9445 48.7045) (width 0.7) (layer B.Cu) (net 9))
 (segment (start 63.9445 48.7045) (end 68.8975 53.6575) (width 0.7) (layer B.Cu) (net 9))
 (segment (start 68.8975 53.6575) (end 68.8975 56.8325) (width 0.7) (layer B.Cu) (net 9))
 (segment (start 68.8975 56.8325) (end 71.0565 58.9915) (width 0.7) (layer B.Cu) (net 9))
 (segment (start 46.2915 47.0535) (end 48.8315 49.5935) (width 0.7) (layer B.Cu) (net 9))
 (segment (start 72.0725 60.0075) (end 71.0565 58.9915) (width 0.7) (layer B.Cu) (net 9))
 (segment (start 72.0725 65.7225) (end 72.0725 60.0075) (width 0.7) (layer B.Cu) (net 9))
 (segment (start 73.9775 67.6275) (end 72.0725 65.7225) (width 0.7) (layer B.Cu) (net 9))
 (segment (start 73.9775 70.0405) (end 73.9775 67.6275) (width 0.7) (layer B.Cu) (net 9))
 (segment (start 71.85914 72.15886) (end 73.9775 70.0405) (width 0.7) (layer B.Cu) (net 9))
 (segment (start 71.85914 72.9615) (end 71.85914 72.15886) (width 0.7) (layer B.Cu) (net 9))
 (segment (start 45.32376 52.05476) (end 45.32376 52.43576) (width 0.7) (layer B.Cu) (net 7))
 (segment (start 49.0855 56.1975) (end 49.7205 56.8325) (width 0.7) (layer B.Cu) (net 7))
 (segment (start 48.768 55.88) (end 49.0855 56.1975) (width 0.7) (layer B.Cu) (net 7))
 (segment (start 45.32376 52.43576) (end 48.768 55.88) (width 0.7) (layer B.Cu) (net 7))
 (segment (start 50.3555 60.1345) (end 52.0065 60.1345) (width 0.7) (layer B.Cu) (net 7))
 (segment (start 49.7205 59.4995) (end 50.3555 60.1345) (width 0.7) (layer B.Cu) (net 7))
 (segment (start 49.7205 56.8325) (end 49.7205 59.4995) (width 0.7) (layer B.Cu) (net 7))
 (segment (start 52.3875 60.5155) (end 52.0065 60.1345) (width 0.7) (layer B.Cu) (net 7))
 (segment (start 57.4675 60.5155) (end 52.3875 60.5155) (width 0.7) (layer B.Cu) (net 7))
 (segment (start 52.0065 60.1345) (end 51.6255 60.1345) (width 0.7) (layer B.Cu) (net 7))
 (segment (start 56.4515 50.4825) (end 51.7525 55.1815) (width 0.7) (layer B.Cu) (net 7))
 (segment (start 51.7525 55.1815) (end 50.1015 55.1815) (width 0.7) (layer B.Cu) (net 7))
 (segment (start 50.1015 55.1815) (end 49.0855 56.1975) (width 0.7) (layer B.Cu) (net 7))
 (segment (start 63.0936 50.4825) (end 56.4515 50.4825) (width 0.7) (layer B.Cu) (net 7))
 (segment (start 65.3415 69.4055) (end 65.3415 67.5005) (width 0.7) (layer B.Cu) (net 5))
 (segment (start 64.7065 66.8655) (end 62.4205 66.8655) (width 0.7) (layer B.Cu) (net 5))
 (segment (start 65.3415 67.5005) (end 64.7065 66.8655) (width 0.7) (layer B.Cu) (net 5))
 (segment (start 56.5785 70.5485) (end 58.4835 70.5485) (width 0.7) (layer B.Cu) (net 5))
 (segment (start 60.0075 69.0245) (end 62.2935 69.0245) (width 0.7) (layer B.Cu) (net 5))
 (segment (start 58.4835 70.5485) (end 60.0075 69.0245) (width 0.7) (layer B.Cu) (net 5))
 (segment (start 62.4205 65.5955) (end 62.4205 66.8655) (width 0.7) (layer B.Cu) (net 5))
 (segment (start 62.4205 66.8655) (end 62.4205 68.8975) (width 0.7) (layer B.Cu) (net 5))
 (segment (start 62.4205 68.8975) (end 62.2935 69.0245) (width 0.7) (layer B.Cu) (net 5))
 (segment (start 57.0865 57.2135) (end 57.0865 55.5625) (width 0.7) (layer B.Cu) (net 5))
 (segment (start 57.0865 55.5625) (end 54.8005 55.5625) (width 0.7) (layer B.Cu) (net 5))
 (segment (start 54.0385 55.5625) (end 52.0065 57.5945) (width 0.7) (layer B.Cu) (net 5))
 (segment (start 54.8005 55.5625) (end 54.0385 55.5625) (width 0.7) (layer B.Cu) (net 5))
 (segment (start 68.7705 69.4055) (end 70.9295 67.2465) (width 0.7) (layer B.Cu) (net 5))
 (segment (start 70.9295 67.2465) (end 70.9295 60.3885) (width 0.7) (layer B.Cu) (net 5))
 (segment (start 70.9295 60.3885) (end 66.8655 56.3245) (width 0.7) (layer B.Cu) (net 5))
 (segment (start 66.8655 56.3245) (end 66.8655 53.9115) (width 0.7) (layer B.Cu) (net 5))
 (segment (start 66.8655 53.9115) (end 65.8495 52.8955) (width 0.7) (layer B.Cu) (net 5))
 (segment (start 65.8495 52.8955) (end 59.7535 52.8955) (width 0.7) (layer B.Cu) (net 5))
 (segment (start 59.7535 52.8955) (end 57.0865 55.5625) (width 0.7) (layer B.Cu) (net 5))
 (segment (start 65.3415 69.4055) (end 68.7705 69.4055) (width 0.7) (layer B.Cu) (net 5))
 (segment (start 68.7705 69.6595) (end 66.1035 72.3265) (width 0.7) (layer B.Cu) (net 5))
 (segment (start 68.7705 69.4055) (end 68.7705 69.6595) (width 0.7) (layer B.Cu) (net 5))
 (segment (start 58.4835 71.1835) (end 58.4835 70.5485) (width 0.7) (layer B.Cu) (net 5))
 (segment (start 56.1975 73.4695) (end 58.4835 71.1835) (width 0.7) (layer B.Cu) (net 5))
 (segment (start 56.1975 73.8505) (end 56.1975 73.4695) (width 0.7) (layer B.Cu) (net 5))
 (segment (start 76.3905 56.4515) (end 76.7715 56.0705) (width 0.7) (layer B.Cu) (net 1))
 (segment (start 76.3905 61.6585) (end 76.3905 56.4515) (width 0.7) (layer B.Cu) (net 1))
 (segment (start 76.98486 62.25286) (end 76.3905 61.6585) (width 0.7) (layer B.Cu) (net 1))
 (segment (start 76.98486 69.1515) (end 76.98486 62.25286) (width 0.7) (layer B.Cu) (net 1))
 (segment (start 73.8505 64.9605) (end 75.1205 66.2305) (width 0.7) (layer B.Cu) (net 13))
 (segment (start 75.1205 66.2305) (end 75.1205 71.2216) (width 0.7) (layer B.Cu) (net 13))
 (segment (start 75.1205 71.2216) (end 76.8604 72.9615) (width 0.7) (layer B.Cu) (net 13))
 (segment (start 73.8505 61.6585) (end 73.8505 64.9605) (width 0.7) (layer B.Cu) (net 13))
 (segment (start 72.3265 48.28286) (end 72.11314 48.0695) (width 0.7) (layer B.Cu) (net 3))
 (segment (start 72.1995 56.7055) (end 73.4695 55.4355) (width 0.7) (layer B.Cu) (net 3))
 (segment (start 73.4695 51.1175) (end 73.4695 49.42586) (width 0.7) (layer B.Cu) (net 3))
 (segment (start 73.4695 55.4355) (end 73.4695 51.1175) (width 0.7) (layer B.Cu) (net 3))
 (segment (start 73.4695 49.42586) (end 72.11314 48.0695) (width 0.7) (layer B.Cu) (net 3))
 (segment (start 71.3105 56.7055) (end 72.1995 56.7055) (width 0.7) (layer B.Cu) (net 3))
 (segment (start 73.4695 50.9905) (end 73.4695 51.1175) (width 0.7) (layer B.Cu) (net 3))
 (segment (start 76.7715 50.9905) (end 73.4695 50.9905) (width 0.7) (layer B.Cu) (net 3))
 (segment (start 68.09486 50.94986) (end 71.3105 54.1655) (width 0.7) (layer B.Cu) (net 14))
 (segment (start 68.09486 50.4825) (end 68.09486 50.94986) (width 0.7) (layer B.Cu) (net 14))
 (segment (start 60.13584 47.0535) (end 57.0865 47.0535) (width 0.7) (layer B.Cu) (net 11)))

